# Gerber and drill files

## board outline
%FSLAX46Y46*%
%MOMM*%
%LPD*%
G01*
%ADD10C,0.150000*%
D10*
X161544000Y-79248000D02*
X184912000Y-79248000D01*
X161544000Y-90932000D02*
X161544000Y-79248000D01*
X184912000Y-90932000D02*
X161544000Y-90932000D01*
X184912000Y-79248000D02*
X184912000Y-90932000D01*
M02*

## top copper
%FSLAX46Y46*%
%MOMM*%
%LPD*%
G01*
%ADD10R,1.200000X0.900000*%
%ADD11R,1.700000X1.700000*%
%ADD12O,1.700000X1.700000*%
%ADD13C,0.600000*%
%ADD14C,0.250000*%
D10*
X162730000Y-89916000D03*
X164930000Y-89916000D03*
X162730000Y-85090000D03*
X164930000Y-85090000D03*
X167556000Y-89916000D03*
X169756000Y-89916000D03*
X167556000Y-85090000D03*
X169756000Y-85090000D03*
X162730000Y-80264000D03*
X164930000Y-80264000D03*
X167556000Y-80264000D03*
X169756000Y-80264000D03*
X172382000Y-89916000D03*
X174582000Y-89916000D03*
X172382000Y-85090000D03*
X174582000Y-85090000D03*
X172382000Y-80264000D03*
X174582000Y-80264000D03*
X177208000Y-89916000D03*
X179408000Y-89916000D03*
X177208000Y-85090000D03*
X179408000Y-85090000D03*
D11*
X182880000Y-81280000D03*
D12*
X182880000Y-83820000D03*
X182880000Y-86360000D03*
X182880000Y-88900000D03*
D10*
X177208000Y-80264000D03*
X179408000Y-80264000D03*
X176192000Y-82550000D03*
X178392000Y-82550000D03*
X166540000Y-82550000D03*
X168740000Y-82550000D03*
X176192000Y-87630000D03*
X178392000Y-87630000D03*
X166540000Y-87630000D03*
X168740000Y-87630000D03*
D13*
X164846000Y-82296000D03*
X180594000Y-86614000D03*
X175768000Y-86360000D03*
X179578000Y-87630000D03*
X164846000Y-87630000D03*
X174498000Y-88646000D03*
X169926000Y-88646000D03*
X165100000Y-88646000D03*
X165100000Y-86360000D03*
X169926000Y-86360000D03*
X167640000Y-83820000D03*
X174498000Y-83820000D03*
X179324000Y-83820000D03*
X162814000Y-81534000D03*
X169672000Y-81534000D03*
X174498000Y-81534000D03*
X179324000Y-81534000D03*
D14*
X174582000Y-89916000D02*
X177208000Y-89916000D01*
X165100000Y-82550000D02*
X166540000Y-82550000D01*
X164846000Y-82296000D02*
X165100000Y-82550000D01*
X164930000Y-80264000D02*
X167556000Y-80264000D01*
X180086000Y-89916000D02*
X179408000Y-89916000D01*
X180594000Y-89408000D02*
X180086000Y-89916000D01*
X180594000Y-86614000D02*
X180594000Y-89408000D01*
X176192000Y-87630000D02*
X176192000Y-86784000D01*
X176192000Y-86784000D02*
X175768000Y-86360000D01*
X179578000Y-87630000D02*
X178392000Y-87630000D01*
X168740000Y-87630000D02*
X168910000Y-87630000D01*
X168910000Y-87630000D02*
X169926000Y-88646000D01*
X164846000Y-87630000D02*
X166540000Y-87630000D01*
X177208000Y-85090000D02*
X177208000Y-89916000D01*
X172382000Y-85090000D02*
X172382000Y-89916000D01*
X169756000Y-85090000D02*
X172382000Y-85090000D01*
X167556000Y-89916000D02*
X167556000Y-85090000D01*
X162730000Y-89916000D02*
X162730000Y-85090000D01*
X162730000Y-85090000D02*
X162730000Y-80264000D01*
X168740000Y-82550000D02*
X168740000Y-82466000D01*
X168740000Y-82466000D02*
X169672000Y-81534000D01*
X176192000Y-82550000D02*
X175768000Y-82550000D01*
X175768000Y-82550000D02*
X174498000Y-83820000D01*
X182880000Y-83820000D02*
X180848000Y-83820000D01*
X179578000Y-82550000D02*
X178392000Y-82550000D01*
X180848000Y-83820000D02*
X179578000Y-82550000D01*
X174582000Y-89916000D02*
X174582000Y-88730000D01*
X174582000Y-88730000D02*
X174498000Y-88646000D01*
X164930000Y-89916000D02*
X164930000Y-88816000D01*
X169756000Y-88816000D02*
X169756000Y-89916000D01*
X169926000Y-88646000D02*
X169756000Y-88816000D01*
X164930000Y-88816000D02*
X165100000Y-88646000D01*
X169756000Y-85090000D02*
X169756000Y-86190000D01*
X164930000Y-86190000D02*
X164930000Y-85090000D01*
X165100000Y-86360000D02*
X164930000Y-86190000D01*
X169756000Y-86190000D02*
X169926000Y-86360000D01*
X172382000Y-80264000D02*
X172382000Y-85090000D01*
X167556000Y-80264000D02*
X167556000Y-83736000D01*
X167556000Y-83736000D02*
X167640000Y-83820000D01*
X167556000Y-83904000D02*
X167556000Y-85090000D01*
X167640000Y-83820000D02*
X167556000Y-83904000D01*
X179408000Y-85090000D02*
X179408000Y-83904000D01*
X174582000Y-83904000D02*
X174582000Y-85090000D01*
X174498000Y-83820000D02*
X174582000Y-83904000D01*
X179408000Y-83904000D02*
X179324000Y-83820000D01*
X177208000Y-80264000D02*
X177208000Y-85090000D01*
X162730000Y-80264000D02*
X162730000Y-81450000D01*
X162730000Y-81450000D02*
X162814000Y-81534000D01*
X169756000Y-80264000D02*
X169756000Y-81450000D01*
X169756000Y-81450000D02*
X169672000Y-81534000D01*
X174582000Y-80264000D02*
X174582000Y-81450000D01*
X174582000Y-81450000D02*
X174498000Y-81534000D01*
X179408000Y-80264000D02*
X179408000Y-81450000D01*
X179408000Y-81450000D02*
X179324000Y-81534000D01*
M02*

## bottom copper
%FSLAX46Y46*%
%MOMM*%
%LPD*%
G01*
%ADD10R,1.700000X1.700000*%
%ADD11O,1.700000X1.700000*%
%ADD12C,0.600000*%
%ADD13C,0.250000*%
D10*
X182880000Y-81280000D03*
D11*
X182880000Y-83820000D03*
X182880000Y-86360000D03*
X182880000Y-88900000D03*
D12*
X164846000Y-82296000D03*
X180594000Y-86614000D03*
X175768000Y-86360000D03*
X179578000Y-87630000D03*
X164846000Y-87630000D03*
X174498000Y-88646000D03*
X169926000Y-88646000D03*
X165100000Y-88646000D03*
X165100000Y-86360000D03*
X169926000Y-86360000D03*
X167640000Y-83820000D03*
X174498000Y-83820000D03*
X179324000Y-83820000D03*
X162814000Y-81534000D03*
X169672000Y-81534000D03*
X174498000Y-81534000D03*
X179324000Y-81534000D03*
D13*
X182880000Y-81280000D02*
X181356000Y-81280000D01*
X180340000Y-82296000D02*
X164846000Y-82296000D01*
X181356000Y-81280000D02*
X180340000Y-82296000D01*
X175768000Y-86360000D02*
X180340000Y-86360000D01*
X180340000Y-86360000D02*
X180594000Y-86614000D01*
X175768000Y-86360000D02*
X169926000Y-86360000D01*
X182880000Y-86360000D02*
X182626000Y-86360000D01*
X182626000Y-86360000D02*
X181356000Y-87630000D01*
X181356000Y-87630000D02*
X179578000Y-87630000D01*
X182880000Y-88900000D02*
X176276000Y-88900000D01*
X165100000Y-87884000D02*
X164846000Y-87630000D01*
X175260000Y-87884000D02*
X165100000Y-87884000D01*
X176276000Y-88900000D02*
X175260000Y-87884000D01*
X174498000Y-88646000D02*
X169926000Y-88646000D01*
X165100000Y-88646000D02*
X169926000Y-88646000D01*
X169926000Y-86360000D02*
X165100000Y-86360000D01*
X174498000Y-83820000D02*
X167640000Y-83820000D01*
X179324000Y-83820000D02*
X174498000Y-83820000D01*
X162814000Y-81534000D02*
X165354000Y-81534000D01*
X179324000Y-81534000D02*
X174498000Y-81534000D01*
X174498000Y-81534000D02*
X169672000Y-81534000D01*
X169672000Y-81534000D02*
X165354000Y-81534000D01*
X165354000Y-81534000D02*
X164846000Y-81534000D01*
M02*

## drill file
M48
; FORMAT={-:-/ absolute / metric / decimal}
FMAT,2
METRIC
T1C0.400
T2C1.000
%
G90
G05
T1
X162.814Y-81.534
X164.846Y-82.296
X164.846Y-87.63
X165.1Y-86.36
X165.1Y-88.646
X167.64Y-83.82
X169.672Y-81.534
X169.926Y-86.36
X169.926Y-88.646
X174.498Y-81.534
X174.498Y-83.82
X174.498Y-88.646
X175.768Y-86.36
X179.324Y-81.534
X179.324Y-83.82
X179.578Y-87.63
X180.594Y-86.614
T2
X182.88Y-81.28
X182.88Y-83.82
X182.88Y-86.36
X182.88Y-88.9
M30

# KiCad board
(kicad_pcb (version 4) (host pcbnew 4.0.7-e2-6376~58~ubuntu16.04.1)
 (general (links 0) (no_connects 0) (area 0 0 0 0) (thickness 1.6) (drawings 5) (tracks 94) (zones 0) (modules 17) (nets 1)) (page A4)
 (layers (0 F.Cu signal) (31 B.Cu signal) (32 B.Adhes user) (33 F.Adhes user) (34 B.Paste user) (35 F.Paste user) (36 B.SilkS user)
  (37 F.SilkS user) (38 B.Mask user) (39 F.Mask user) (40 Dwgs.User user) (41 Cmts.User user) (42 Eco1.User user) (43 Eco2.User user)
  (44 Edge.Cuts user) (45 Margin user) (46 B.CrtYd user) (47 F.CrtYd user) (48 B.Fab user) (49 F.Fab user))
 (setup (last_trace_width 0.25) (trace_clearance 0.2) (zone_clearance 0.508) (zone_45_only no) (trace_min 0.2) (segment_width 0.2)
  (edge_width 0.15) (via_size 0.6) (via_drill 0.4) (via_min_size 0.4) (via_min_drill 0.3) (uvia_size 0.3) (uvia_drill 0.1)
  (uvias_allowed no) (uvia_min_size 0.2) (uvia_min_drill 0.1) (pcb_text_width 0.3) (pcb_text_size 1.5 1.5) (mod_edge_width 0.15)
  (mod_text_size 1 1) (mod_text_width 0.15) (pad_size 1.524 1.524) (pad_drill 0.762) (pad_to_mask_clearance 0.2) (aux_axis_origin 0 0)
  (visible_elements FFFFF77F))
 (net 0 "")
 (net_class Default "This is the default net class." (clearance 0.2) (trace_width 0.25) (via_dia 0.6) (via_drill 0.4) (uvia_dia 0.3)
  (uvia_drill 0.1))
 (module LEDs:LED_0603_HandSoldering (layer F.Cu) (at 163.83 89.916)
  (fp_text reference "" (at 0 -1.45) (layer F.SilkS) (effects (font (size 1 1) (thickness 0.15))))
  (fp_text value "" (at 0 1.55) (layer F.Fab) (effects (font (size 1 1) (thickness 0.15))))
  (pad 1 smd rect (at -1.1 0) (size 1.2 0.9) (layers F.Cu F.Paste F.Mask))
  (pad 2 smd rect (at 1.1 0) (size 1.2 0.9) (layers F.Cu F.Paste F.Mask)))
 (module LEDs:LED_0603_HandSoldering (layer F.Cu) (at 163.83 85.09)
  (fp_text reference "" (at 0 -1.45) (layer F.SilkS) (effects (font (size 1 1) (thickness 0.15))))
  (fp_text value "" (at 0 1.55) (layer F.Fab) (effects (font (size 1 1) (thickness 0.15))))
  (pad 1 smd rect (at -1.1 0) (size 1.2 0.9) (layers F.Cu F.Paste F.Mask))
  (pad 2 smd rect (at 1.1 0) (size 1.2 0.9) (layers F.Cu F.Paste F.Mask)))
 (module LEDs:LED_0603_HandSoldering (layer F.Cu) (at 168.656 89.916)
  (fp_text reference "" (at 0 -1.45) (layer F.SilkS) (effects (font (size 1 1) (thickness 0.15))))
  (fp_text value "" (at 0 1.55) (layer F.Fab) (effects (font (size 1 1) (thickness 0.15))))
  (pad 1 smd rect (at -1.1 0) (size 1.2 0.9) (layers F.Cu F.Paste F.Mask))
  (pad 2 smd rect (at 1.1 0) (size 1.2 0.9) (layers F.Cu F.Paste F.Mask)))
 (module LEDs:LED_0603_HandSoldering (layer F.Cu) (at 168.656 85.09)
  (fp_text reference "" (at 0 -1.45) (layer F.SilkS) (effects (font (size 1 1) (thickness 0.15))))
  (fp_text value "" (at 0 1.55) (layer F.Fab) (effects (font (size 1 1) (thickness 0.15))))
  (pad 1 smd rect (at -1.1 0) (size 1.2 0.9) (layers F.Cu F.Paste F.Mask))
  (pad 2 smd rect (at 1.1 0) (size 1.2 0.9) (layers F.Cu F.Paste F.Mask)))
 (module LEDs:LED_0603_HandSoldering (layer F.Cu) (at 163.83 80.264)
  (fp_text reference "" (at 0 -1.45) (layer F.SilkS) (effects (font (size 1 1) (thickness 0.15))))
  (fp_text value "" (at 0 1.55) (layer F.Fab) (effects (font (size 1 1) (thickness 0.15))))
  (pad 1 smd rect (at -1.1 0) (size 1.2 0.9) (layers F.Cu F.Paste F.Mask))
  (pad 2 smd rect (at 1.1 0) (size 1.2 0.9) (layers F.Cu F.Paste F.Mask)))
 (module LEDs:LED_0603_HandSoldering (layer F.Cu) (at 168.656 80.264)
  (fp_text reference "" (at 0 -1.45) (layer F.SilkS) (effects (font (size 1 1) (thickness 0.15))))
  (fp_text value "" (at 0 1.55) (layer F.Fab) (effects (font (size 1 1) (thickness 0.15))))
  (pad 1 smd rect (at -1.1 0) (size 1.2 0.9) (layers F.Cu F.Paste F.Mask))
  (pad 2 smd rect (at 1.1 0) (size 1.2 0.9) (layers F.Cu F.Paste F.Mask)))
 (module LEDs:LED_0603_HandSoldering (layer F.Cu) (at 173.482 89.916)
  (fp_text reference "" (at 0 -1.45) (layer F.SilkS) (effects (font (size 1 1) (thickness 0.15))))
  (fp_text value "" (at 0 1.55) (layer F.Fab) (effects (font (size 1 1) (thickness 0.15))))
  (pad 1 smd rect (at -1.1 0) (size 1.2 0.9) (layers F.Cu F.Paste F.Mask))
  (pad 2 smd rect (at 1.1 0) (size 1.2 0.9) (layers F.Cu F.Paste F.Mask)))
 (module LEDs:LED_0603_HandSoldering (layer F.Cu) (at 173.482 85.09)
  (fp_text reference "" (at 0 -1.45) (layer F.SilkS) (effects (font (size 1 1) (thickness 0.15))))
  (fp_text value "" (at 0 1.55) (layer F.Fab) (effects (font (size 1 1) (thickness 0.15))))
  (pad 1 smd rect (at -1.1 0) (size 1.2 0.9) (layers F.Cu F.Paste F.Mask))
  (pad 2 smd rect (at 1.1 0) (size 1.2 0.9) (layers F.Cu F.Paste F.Mask)))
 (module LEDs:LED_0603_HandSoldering (layer F.Cu) (at 173.482 80.264)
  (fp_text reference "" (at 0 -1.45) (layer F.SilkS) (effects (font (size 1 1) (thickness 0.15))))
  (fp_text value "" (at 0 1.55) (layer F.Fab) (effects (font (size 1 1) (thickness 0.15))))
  (pad 1 smd rect (at -1.1 0) (size 1.2 0.9) (layers F.Cu F.Paste F.Mask))
  (pad 2 smd rect (at 1.1 0) (size 1.2 0.9) (layers F.Cu F.Paste F.Mask)))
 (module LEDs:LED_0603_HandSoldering (layer F.Cu) (at 178.308 89.916)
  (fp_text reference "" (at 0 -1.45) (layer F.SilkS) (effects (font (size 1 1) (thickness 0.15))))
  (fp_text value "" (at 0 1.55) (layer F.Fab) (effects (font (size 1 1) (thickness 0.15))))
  (pad 1 smd rect (at -1.1 0) (size 1.2 0.9) (layers F.Cu F.Paste F.Mask))
  (pad 2 smd rect (at 1.1 0) (size 1.2 0.9) (layers F.Cu F.Paste F.Mask)))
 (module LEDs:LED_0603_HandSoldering (layer F.Cu) (at 178.308 85.09)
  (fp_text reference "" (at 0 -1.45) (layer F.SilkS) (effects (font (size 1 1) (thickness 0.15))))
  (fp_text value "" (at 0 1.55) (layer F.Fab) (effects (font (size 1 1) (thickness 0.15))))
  (pad 1 smd rect (at -1.1 0) (size 1.2 0.9) (layers F.Cu F.Paste F.Mask))
  (pad 2 smd rect (at 1.1 0) (size 1.2 0.9) (layers F.Cu F.Paste F.Mask)))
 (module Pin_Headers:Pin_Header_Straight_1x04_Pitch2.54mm (layer F.Cu) (at 182.88 81.28)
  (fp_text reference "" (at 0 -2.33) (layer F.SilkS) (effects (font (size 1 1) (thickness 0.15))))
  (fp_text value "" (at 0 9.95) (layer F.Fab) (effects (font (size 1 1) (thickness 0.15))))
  (pad 1 thru_hole rect (at 0 0) (size 1.7 1.7) (drill 1) (layers *.Cu *.Mask))
  (pad 2 thru_hole oval (at 0 2.54) (size 1.7 1.7) (drill 1) (layers *.Cu *.Mask))
  (pad 3 thru_hole oval (at 0 5.08) (size 1.7 1.7) (drill 1) (layers *.Cu *.Mask))
  (pad 4 thru_hole oval (at 0 7.62) (size 1.7 1.7) (drill 1) (layers *.Cu *.Mask)))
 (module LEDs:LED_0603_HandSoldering (layer F.Cu) (at 178.308 80.264)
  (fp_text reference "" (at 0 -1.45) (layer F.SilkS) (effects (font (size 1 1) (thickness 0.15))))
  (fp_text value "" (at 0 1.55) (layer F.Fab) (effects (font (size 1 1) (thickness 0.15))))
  (pad 1 smd rect (at -1.1 0) (size 1.2 0.9) (layers F.Cu F.Paste F.Mask))
  (pad 2 smd rect (at 1.1 0) (size 1.2 0.9) (layers F.Cu F.Paste F.Mask)))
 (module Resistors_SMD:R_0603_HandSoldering (layer F.Cu) (at 177.292 82.55)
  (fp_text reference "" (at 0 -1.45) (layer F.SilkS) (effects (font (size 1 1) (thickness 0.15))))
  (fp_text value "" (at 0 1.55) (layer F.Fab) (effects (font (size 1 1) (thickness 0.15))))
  (pad 1 smd rect (at -1.1 0) (size 1.2 0.9) (layers F.Cu F.Paste F.Mask))
  (pad 2 smd rect (at 1.1 0) (size 1.2 0.9) (layers F.Cu F.Paste F.Mask)))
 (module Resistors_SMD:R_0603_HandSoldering (layer F.Cu) (at 167.64 82.55)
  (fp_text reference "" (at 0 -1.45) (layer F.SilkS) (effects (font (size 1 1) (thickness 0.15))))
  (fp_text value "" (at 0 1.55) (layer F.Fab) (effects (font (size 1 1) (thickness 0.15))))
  (pad 1 smd rect (at -1.1 0) (size 1.2 0.9) (layers F.Cu F.Paste F.Mask))
  (pad 2 smd rect (at 1.1 0) (size 1.2 0.9) (layers F.Cu F.Paste F.Mask)))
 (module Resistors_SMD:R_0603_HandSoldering (layer F.Cu) (at 177.292 87.63)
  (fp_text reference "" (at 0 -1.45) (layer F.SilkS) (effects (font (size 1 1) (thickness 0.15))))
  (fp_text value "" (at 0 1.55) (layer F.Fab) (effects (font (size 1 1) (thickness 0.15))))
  (pad 1 smd rect (at -1.1 0) (size 1.2 0.9) (layers F.Cu F.Paste F.Mask))
  (pad 2 smd rect (at 1.1 0) (size 1.2 0.9) (layers F.Cu F.Paste F.Mask)))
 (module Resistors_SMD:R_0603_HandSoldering (layer F.Cu) (at 167.64 87.63)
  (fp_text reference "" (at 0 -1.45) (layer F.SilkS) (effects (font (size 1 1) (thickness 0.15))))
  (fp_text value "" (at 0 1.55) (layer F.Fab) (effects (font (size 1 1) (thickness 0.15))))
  (pad 1 smd rect (at -1.1 0) (size 1.2 0.9) (layers F.Cu F.Paste F.Mask))
  (pad 2 smd rect (at 1.1 0) (size 1.2 0.9) (layers F.Cu F.Paste F.Mask)))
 (gr_line (start 161.544 79.248) (end 184.912 79.248) (angle 90) (layer Edge.Cuts) (width 0.15))
 (gr_line (start 161.544 90.932) (end 161.544 79.248) (angle 90) (layer Edge.Cuts) (width 0.15))
 (gr_line (start 184.912 90.932) (end 161.544 90.932) (angle 90) (layer Edge.Cuts) (width 0.15))
 (gr_line (start 184.912 79.248) (end 184.912 90.932) (angle 90) (layer Edge.Cuts) (width 0.15))
 (segment (start 174.582 89.916) (end 177.208 89.916) (width 0.25) (layer F.Cu) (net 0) (status C00000))
 (segment (start 182.88 81.28) (end 181.356 81.28) (width 0.25) (layer B.Cu) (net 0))
 (segment (start 165.1 82.55) (end 166.54 82.55) (width 0.25) (layer F.Cu) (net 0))
 (segment (start 164.846 82.296) (end 165.1 82.55) (width 0.25) (layer F.Cu) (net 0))
 (via (at 164.846 82.296) (size 0.6) (drill 0.4) (layers F.Cu B.Cu) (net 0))
 (segment (start 180.34 82.296) (end 164.846 82.296) (width 0.25) (layer B.Cu) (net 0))
 (segment (start 181.356 81.28) (end 180.34 82.296) (width 0.25) (layer B.Cu) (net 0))
 (segment (start 164.93 80.264) (end 167.556 80.264) (width 0.25) (layer F.Cu) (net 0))
 (segment (start 175.768 86.36) (end 180.34 86.36) (width 0.25) (layer B.Cu) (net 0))
 (segment (start 180.086 89.916) (end 179.408 89.916) (width 0.25) (layer F.Cu) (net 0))
 (segment (start 180.594 89.408) (end 180.086 89.916) (width 0.25) (layer F.Cu) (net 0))
 (segment (start 180.594 86.614) (end 180.594 89.408) (width 0.25) (layer F.Cu) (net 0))
 (via (at 180.594 86.614) (size 0.6) (drill 0.4) (layers F.Cu B.Cu) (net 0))
 (segment (start 180.34 86.36) (end 180.594 86.614) (width 0.25) (layer B.Cu) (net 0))
 (segment (start 176.192 87.63) (end 176.192 86.784) (width 0.25) (layer F.Cu) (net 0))
 (segment (start 175.768 86.36) (end 169.926 86.36) (width 0.25) (layer B.Cu) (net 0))
 (via (at 175.768 86.36) (size 0.6) (drill 0.4) (layers F.Cu B.Cu) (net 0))
 (segment (start 176.192 86.784) (end 175.768 86.36) (width 0.25) (layer F.Cu) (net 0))
 (segment (start 182.88 86.36) (end 182.626 86.36) (width 0.25) (layer B.Cu) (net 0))
 (segment (start 182.626 86.36) (end 181.356 87.63) (width 0.25) (layer B.Cu) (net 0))
 (segment (start 181.356 87.63) (end 179.578 87.63) (width 0.25) (layer B.Cu) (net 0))
 (via (at 179.578 87.63) (size 0.6) (drill 0.4) (layers F.Cu B.Cu) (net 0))
 (segment (start 179.578 87.63) (end 178.392 87.63) (width 0.25) (layer F.Cu) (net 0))
 (segment (start 168.74 87.63) (end 168.91 87.63) (width 0.25) (layer F.Cu) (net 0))
 (segment (start 168.91 87.63) (end 169.926 88.646) (width 0.25) (layer F.Cu) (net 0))
 (segment (start 182.88 88.9) (end 176.276 88.9) (width 0.25) (layer B.Cu) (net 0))
 (segment (start 164.846 87.63) (end 166.54 87.63) (width 0.25) (layer F.Cu) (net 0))
 (via (at 164.846 87.63) (size 0.6) (drill 0.4) (layers F.Cu B.Cu) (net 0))
 (segment (start 165.1 87.884) (end 164.846 87.63) (width 0.25) (layer B.Cu) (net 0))
 (segment (start 175.26 87.884) (end 165.1 87.884) (width 0.25) (layer B.Cu) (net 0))
 (segment (start 176.276 88.9) (end 175.26 87.884) (width 0.25) (layer B.Cu) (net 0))
 (segment (start 177.208 85.09) (end 177.208 89.916) (width 0.25) (layer F.Cu) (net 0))
 (segment (start 172.382 85.09) (end 172.382 89.916) (width 0.25) (layer F.Cu) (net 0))
 (segment (start 169.756 85.09) (end 172.382 85.09) (width 0.25) (layer F.Cu) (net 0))
 (segment (start 167.556 89.916) (end 167.556 85.09) (width 0.25) (layer F.Cu) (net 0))
 (segment (start 162.73 89.916) (end 162.73 85.09) (width 0.25) (layer F.Cu) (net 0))
 (segment (start 162.73 85.09) (end 162.73 80.264) (width 0.25) (layer F.Cu) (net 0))
 (segment (start 168.74 82.55) (end 168.74 82.466) (width 0.25) (layer F.Cu) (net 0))
 (segment (start 168.74 82.466) (end 169.672 81.534) (width 0.25) (layer F.Cu) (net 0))
 (segment (start 176.192 82.55) (end 175.768 82.55) (width 0.25) (layer F.Cu) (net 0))
 (segment (start 175.768 82.55) (end 174.498 83.82) (width 0.25) (layer F.Cu) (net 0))
 (segment (start 182.88 83.82) (end 180.848 83.82) (width 0.25) (layer F.Cu) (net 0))
 (segment (start 179.578 82.55) (end 178.392 82.55) (width 0.25) (layer F.Cu) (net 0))
 (segment (start 180.848 83.82) (end 179.578 82.55) (width 0.25) (layer F.Cu) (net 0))
 (segment (start 174.582 89.916) (end 174.582 88.73) (width 0.25) (layer F.Cu) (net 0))
 (segment (start 174.498 88.646) (end 169.926 88.646) (width 0.25) (layer B.Cu) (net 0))
 (via (at 174.498 88.646) (size 0.6) (drill 0.4) (layers F.Cu B.Cu) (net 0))
 (segment (start 174.582 88.73) (end 174.498 88.646) (width 0.25) (layer F.Cu) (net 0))
 (segment (start 164.93 89.916) (end 164.93 88.816) (width 0.25) (layer F.Cu) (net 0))
 (segment (start 169.756 88.816) (end 169.756 89.916) (width 0.25) (layer F.Cu) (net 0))
 (segment (start 169.926 88.646) (end 169.756 88.816) (width 0.25) (layer F.Cu) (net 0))
 (via (at 169.926 88.646) (size 0.6) (drill 0.4) (layers F.Cu B.Cu) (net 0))
 (segment (start 165.1 88.646) (end 169.926 88.646) (width 0.25) (layer B.Cu) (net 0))
 (via (at 165.1 88.646) (size 0.6) (drill 0.4) (layers F.Cu B.Cu) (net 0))
 (segment (start 164.93 88.816) (end 165.1 88.646) (width 0.25) (layer F.Cu) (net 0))
 (segment (start 169.756 85.09) (end 169.756 86.19) (width 0.25) (layer F.Cu) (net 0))
 (segment (start 164.93 86.19) (end 164.93 85.09) (width 0.25) (layer F.Cu) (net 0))
 (segment (start 165.1 86.36) (end 164.93 86.19) (width 0.25) (layer F.Cu) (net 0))
 (via (at 165.1 86.36) (size 0.6) (drill 0.4) (layers F.Cu B.Cu) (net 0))
 (segment (start 169.926 86.36) (end 165.1 86.36) (width 0.25) (layer B.Cu) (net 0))
 (via (at 169.926 86.36) (size 0.6) (drill 0.4) (layers F.Cu B.Cu) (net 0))
 (segment (start 169.756 86.19) (end 169.926 86.36) (width 0.25) (layer F.Cu) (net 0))
 (segment (start 172.382 80.264) (end 172.382 85.09) (width 0.25) (layer F.Cu) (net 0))
 (segment (start 167.556 80.264) (end 167.556 83.736) (width 0.25) (layer F.Cu) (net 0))
 (segment (start 167.556 83.736) (end 167.64 83.82) (width 0.25) (layer F.Cu) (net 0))
 (segment (start 174.498 83.82) (end 167.64 83.82) (width 0.25) (layer B.Cu) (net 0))
 (segment (start 167.556 83.904) (end 167.556 85.09) (width 0.25) (layer F.Cu) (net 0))
 (segment (start 167.64 83.82) (end 167.556 83.904) (width 0.25) (layer F.Cu) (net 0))
 (via (at 167.64 83.82) (size 0.6) (drill 0.4) (layers F.Cu B.Cu) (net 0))
 (segment (start 179.408 85.09) (end 179.408 83.904) (width 0.25) (layer F.Cu) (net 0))
 (segment (start 174.582 83.904) (end 174.582 85.09) (width 0.25) (layer F.Cu) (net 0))
 (segment (start 174.498 83.82) (end 174.582 83.904) (width 0.25) (layer F.Cu) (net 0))
 (via (at 174.498 83.82) (size 0.6) (drill 0.4) (layers F.Cu B.Cu) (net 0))
 (segment (start 179.324 83.82) (end 174.498 83.82) (width 0.25) (layer B.Cu) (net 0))
 (via (at 179.324 83.82) (size 0.6) (drill 0.4) (layers F.Cu B.Cu) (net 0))
 (segment (start 179.408 83.904) (end 179.324 83.82) (width 0.25) (layer F.Cu) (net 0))
 (segment (start 177.208 80.264) (end 177.208 85.09) (width 0.25) (layer F.Cu) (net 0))
 (segment (start 162.73 80.264) (end 162.73 81.45) (width 0.25) (layer F.Cu) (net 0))
 (segment (start 162.814 81.534) (end 165.354 81.534) (width 0.25) (layer B.Cu) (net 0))
 (via (at 162.814 81.534) (size 0.6) (drill 0.4) (layers F.Cu B.Cu) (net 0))
 (segment (start 162.73 81.45) (end 162.814 81.534) (width 0.25) (layer F.Cu) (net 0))
 (segment (start 169.756 80.264) (end 169.756 81.45) (width 0.25) (layer F.Cu) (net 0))
 (via (at 169.672 81.534) (size 0.6) (drill 0.4) (layers F.Cu B.Cu) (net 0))
 (segment (start 169.756 81.45) (end 169.672 81.534) (width 0.25) (layer F.Cu) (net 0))
 (segment (start 174.582 80.264) (end 174.582 81.45) (width 0.25) (layer F.Cu) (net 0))
 (via (at 174.498 81.534) (size 0.6) (drill 0.4) (layers F.Cu B.Cu) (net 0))
 (segment (start 174.582 81.45) (end 174.498 81.534) (width 0.25) (layer F.Cu) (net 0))
 (segment (start 179.408 80.264) (end 179.408 81.45) (width 0.25) (layer F.Cu) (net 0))
 (segment (start 179.324 81.534) (end 174.498 81.534) (width 0.25) (layer B.Cu) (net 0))
 (segment (start 174.498 81.534) (end 169.672 81.534) (width 0.25) (layer B.Cu) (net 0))
 (segment (start 169.672 81.534) (end 165.354 81.534) (width 0.25) (layer B.Cu) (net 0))
 (segment (start 165.354 81.534) (end 164.846 81.534) (width 0.25) (layer B.Cu) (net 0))
 (via (at 179.324 81.534) (size 0.6) (drill 0.4) (layers F.Cu B.Cu) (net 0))
 (segment (start 179.408 81.45) (end 179.324 81.534) (width 0.25) (layer F.Cu) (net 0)))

